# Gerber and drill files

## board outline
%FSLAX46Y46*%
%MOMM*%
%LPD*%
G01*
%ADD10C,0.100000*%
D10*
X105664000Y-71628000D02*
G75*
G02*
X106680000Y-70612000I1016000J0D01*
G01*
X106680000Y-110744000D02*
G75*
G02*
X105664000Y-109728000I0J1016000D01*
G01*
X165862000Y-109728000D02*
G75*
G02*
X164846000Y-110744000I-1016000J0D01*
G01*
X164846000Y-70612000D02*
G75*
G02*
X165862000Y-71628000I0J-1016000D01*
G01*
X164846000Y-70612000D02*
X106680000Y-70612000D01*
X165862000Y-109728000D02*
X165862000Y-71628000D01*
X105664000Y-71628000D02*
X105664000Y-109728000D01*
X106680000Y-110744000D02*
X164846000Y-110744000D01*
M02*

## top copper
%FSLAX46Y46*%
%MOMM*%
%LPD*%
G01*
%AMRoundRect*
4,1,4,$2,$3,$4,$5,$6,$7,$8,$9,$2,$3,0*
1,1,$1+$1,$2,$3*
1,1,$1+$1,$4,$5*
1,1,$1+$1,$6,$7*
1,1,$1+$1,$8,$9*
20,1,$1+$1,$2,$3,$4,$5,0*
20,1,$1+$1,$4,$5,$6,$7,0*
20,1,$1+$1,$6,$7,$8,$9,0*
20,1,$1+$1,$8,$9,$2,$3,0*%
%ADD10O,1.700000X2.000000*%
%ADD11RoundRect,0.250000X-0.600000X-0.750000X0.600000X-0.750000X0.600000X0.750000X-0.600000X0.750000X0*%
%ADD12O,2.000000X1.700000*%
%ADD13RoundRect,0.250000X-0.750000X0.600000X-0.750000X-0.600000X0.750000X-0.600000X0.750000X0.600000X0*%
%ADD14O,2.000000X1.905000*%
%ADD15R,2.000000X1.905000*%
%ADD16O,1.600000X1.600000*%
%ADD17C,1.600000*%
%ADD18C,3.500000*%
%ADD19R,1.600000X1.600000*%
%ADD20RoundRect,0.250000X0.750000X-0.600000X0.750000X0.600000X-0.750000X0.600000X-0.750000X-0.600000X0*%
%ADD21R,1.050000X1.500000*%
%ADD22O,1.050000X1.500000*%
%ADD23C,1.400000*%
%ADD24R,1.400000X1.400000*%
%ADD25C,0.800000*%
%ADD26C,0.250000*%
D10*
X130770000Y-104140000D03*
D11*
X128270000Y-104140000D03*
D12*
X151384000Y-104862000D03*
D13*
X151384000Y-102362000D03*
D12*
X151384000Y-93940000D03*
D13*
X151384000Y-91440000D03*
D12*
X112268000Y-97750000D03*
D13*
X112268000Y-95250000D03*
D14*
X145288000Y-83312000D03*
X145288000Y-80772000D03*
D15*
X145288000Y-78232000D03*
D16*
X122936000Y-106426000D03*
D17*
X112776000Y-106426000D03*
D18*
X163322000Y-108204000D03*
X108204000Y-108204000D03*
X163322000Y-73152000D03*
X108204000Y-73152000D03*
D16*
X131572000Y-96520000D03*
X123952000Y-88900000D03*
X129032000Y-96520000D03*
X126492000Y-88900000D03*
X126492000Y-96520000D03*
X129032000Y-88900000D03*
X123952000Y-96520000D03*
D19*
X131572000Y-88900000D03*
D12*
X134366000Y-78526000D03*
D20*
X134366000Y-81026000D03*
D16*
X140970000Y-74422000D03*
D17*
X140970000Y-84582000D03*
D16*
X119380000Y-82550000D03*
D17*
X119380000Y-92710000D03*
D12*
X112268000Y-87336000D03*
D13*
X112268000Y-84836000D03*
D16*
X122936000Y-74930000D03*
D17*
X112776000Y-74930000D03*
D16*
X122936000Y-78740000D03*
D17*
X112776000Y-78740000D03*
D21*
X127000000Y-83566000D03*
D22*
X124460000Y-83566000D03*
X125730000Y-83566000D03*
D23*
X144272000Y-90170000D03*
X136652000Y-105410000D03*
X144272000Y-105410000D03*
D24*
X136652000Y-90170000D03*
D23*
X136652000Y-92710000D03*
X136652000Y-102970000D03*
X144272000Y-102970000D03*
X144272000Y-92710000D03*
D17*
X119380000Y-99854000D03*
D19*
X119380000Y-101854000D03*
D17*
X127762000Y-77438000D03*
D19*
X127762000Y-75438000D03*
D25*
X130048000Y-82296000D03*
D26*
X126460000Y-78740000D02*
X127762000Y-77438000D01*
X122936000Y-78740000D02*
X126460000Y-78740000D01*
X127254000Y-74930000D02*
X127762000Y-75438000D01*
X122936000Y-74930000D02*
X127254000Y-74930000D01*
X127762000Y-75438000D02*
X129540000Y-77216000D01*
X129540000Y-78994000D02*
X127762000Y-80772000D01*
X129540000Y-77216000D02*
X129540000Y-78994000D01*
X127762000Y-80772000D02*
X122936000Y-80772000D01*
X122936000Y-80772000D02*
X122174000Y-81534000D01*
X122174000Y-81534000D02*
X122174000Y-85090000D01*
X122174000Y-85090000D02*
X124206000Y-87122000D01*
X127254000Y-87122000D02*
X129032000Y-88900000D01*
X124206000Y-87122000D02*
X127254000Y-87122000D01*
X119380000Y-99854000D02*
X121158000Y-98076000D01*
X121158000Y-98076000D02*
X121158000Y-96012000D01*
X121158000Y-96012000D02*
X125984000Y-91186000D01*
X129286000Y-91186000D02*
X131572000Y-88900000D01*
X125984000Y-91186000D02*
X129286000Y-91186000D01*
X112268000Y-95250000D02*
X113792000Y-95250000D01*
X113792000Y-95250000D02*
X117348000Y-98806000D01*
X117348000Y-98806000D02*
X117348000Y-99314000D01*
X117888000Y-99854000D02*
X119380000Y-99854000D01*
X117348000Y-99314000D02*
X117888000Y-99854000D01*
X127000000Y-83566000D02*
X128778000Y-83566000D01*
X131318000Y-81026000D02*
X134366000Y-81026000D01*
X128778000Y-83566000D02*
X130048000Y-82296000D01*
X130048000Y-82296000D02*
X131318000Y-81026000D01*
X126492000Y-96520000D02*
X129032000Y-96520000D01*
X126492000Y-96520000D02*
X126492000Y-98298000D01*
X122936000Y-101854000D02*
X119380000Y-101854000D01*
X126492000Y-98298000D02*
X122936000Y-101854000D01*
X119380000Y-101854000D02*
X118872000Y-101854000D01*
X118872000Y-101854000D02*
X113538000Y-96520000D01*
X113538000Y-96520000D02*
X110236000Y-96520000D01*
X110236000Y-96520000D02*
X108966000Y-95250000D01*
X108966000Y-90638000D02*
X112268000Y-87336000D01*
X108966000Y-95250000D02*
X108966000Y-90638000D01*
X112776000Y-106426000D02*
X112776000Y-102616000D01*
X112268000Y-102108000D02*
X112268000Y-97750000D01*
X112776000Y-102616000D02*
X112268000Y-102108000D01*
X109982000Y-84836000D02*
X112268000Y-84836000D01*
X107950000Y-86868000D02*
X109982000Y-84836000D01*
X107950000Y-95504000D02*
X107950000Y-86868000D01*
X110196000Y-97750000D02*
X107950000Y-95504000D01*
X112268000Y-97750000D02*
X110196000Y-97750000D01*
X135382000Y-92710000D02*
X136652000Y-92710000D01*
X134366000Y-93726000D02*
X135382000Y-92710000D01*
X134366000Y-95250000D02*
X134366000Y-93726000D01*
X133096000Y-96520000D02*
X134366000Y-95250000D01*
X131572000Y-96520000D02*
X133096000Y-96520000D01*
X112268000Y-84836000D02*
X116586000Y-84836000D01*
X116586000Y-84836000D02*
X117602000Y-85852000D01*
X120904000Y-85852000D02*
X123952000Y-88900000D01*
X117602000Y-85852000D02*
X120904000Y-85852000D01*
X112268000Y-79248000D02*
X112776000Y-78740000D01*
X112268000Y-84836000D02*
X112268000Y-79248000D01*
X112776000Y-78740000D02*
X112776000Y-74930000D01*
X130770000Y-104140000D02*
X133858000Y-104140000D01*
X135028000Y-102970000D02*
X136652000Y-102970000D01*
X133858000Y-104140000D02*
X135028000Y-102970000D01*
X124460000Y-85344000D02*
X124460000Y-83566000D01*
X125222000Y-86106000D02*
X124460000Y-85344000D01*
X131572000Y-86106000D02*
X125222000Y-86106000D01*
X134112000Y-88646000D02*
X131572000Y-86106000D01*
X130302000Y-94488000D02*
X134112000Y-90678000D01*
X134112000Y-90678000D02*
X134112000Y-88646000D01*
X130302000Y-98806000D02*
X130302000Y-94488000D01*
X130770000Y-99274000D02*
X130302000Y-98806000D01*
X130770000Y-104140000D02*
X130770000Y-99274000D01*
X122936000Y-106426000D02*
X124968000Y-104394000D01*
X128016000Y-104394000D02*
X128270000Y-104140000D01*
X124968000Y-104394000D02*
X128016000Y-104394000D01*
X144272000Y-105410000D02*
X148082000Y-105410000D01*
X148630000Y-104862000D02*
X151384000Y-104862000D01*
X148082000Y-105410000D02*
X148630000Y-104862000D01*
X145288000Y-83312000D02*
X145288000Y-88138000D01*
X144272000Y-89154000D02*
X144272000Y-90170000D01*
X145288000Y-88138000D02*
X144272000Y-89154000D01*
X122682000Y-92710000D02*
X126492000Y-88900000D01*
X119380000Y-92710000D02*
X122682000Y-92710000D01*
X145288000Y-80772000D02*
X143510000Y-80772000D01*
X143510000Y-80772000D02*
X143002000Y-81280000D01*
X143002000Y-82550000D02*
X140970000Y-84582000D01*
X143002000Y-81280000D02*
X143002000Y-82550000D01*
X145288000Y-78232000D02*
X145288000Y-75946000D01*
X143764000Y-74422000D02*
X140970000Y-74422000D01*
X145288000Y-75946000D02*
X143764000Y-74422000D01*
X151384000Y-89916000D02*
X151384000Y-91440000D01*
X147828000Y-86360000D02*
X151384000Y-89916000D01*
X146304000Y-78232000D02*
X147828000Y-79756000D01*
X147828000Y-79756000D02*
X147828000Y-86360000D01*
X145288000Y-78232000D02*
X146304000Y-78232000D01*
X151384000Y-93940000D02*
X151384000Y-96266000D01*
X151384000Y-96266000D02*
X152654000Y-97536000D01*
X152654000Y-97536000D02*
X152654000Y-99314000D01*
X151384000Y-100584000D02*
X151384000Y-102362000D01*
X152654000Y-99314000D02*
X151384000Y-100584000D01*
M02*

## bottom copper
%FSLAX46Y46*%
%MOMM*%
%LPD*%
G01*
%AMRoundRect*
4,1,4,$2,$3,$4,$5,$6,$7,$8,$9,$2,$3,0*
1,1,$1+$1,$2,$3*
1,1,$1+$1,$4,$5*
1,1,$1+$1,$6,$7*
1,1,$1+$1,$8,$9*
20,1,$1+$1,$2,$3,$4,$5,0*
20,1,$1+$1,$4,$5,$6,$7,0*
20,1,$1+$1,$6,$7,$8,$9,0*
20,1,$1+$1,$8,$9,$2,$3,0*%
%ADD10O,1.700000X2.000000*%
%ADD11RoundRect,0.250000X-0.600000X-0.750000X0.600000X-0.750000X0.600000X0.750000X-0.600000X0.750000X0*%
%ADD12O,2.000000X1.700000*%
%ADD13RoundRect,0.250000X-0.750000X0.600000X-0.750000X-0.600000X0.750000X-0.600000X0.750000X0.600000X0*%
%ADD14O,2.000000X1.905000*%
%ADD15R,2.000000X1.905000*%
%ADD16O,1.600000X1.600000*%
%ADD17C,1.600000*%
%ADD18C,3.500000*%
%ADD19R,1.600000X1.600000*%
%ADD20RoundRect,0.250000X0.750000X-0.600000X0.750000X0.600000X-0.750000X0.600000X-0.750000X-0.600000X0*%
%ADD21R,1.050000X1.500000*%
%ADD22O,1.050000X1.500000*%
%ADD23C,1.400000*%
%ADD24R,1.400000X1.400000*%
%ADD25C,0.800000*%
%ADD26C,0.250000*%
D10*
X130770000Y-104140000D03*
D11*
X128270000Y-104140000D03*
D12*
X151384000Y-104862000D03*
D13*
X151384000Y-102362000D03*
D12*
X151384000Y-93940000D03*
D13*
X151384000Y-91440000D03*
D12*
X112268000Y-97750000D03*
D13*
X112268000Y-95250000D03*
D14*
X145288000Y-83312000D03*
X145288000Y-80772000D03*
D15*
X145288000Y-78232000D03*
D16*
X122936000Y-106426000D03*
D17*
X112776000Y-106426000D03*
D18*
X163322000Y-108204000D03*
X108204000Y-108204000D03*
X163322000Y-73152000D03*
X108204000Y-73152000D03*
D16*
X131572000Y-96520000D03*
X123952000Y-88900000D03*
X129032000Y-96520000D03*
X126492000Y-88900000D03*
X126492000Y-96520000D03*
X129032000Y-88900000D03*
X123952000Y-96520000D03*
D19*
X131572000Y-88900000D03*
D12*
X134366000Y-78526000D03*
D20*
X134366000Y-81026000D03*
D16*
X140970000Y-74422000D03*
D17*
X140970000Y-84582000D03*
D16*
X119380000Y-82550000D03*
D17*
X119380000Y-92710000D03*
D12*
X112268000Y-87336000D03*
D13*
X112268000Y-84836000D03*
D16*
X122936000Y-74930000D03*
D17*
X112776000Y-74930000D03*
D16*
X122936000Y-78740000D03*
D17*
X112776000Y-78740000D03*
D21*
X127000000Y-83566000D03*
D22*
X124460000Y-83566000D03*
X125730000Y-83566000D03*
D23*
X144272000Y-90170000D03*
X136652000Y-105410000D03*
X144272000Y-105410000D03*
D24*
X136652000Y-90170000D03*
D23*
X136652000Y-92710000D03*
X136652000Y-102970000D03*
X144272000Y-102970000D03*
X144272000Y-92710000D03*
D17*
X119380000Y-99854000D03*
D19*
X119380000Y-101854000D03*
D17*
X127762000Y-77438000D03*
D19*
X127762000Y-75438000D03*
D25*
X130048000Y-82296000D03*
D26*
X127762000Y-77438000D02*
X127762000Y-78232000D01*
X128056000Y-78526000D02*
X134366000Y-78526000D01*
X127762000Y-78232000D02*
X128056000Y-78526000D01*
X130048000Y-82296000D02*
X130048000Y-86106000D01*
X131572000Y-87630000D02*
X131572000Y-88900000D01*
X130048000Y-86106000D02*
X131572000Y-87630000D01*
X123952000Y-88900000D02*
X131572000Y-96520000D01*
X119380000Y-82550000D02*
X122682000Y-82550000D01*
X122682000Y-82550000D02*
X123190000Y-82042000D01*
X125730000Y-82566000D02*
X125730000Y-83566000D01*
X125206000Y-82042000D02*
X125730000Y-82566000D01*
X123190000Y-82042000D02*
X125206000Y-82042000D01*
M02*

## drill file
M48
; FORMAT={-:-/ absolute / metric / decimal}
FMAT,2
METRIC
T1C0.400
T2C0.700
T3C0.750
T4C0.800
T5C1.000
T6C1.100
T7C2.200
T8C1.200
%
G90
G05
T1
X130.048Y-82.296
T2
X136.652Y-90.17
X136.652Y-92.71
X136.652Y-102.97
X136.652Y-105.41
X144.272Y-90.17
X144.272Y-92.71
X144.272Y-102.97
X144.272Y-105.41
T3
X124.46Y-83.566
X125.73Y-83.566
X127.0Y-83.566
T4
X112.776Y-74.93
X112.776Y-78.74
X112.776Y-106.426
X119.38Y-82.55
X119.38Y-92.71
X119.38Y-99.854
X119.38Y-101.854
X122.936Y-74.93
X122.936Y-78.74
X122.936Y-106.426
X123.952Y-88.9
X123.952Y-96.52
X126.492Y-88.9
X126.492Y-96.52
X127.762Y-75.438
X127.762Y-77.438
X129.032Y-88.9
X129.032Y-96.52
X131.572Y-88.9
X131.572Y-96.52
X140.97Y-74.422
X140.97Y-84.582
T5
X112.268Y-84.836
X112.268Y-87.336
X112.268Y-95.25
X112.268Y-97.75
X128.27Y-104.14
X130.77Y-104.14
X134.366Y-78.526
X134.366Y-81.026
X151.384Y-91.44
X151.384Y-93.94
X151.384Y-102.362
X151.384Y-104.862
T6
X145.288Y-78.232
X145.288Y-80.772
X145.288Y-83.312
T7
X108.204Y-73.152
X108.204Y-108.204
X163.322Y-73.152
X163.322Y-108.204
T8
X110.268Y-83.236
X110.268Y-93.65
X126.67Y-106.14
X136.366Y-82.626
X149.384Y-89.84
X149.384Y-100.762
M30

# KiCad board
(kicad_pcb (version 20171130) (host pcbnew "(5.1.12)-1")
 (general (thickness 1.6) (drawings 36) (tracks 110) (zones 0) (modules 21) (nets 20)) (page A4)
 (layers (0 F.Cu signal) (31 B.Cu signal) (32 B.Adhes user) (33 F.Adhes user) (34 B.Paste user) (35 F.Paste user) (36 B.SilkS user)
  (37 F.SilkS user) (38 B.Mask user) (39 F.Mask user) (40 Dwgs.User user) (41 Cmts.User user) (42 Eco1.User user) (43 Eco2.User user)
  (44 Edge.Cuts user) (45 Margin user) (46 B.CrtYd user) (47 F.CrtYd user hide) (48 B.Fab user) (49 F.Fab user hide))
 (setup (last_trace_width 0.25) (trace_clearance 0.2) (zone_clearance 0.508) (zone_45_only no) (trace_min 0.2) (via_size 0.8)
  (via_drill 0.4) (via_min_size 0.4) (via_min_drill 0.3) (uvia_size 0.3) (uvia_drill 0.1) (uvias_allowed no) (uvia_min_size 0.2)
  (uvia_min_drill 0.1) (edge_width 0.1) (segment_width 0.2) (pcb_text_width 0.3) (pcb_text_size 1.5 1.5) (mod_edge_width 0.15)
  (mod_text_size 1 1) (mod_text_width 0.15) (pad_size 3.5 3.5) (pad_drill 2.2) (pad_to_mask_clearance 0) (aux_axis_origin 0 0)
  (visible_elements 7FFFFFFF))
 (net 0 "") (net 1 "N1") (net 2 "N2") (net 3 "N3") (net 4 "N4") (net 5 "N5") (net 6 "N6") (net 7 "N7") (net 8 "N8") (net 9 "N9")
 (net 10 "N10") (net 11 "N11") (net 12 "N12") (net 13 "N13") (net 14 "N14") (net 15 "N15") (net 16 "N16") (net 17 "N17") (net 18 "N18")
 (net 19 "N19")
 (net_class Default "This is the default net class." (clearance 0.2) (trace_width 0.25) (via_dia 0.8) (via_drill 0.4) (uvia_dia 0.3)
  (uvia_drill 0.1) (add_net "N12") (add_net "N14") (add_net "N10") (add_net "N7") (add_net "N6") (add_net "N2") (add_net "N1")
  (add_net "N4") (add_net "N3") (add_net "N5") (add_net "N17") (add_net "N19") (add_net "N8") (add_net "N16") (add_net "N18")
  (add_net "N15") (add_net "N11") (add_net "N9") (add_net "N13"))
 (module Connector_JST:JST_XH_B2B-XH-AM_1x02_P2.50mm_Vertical (layer F.Cu) (at 128.27 104.14)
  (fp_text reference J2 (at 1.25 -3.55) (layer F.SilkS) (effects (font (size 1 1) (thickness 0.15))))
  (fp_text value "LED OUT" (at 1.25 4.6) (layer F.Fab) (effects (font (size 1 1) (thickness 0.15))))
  (pad "" np_thru_hole circle (at -1.6 2) (size 1.2 1.2) (drill 1.2) (layers *.Cu *.Mask))
  (pad 2 thru_hole oval (at 2.5 0) (size 1.7 2) (drill 1) (layers *.Cu *.Mask) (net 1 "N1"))
  (pad 1 thru_hole roundrect (at 0 0) (size 1.7 2) (drill 1) (layers *.Cu *.Mask) (roundrect_rratio 0.147059) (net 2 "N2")))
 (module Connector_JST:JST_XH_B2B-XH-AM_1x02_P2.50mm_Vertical (layer F.Cu) (at 151.384 102.362 270)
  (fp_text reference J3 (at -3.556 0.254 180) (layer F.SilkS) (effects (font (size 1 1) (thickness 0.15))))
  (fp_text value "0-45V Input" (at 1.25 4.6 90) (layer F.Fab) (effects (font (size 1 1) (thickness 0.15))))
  (pad "" np_thru_hole circle (at -1.6 2 270) (size 1.2 1.2) (drill 1.2) (layers *.Cu *.Mask))
  (pad 2 thru_hole oval (at 2.5 0 270) (size 1.7 2) (drill 1) (layers *.Cu *.Mask) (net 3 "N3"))
  (pad 1 thru_hole roundrect (at 0 0 270) (size 1.7 2) (drill 1) (layers *.Cu *.Mask) (roundrect_rratio 0.147059) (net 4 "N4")))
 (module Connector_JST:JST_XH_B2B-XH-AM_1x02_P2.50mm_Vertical (layer F.Cu) (at 151.384 91.44 270)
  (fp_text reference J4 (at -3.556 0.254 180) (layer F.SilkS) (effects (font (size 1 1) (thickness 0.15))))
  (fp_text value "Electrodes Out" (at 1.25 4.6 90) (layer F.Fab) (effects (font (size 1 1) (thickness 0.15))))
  (pad "" np_thru_hole circle (at -1.6 2 270) (size 1.2 1.2) (drill 1.2) (layers *.Cu *.Mask))
  (pad 2 thru_hole oval (at 2.5 0 270) (size 1.7 2) (drill 1) (layers *.Cu *.Mask) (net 4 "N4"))
  (pad 1 thru_hole roundrect (at 0 0 270) (size 1.7 2) (drill 1) (layers *.Cu *.Mask) (roundrect_rratio 0.147059) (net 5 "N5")))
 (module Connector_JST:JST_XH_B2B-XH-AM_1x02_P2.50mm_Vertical (layer F.Cu) (at 112.268 95.25 270)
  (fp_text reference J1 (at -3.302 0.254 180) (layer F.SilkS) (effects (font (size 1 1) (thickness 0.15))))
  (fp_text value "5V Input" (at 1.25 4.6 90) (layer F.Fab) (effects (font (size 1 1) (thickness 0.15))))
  (pad "" np_thru_hole circle (at -1.6 2 270) (size 1.2 1.2) (drill 1.2) (layers *.Cu *.Mask))
  (pad 2 thru_hole oval (at 2.5 0 270) (size 1.7 2) (drill 1) (layers *.Cu *.Mask) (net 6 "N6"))
  (pad 1 thru_hole roundrect (at 0 0 270) (size 1.7 2) (drill 1) (layers *.Cu *.Mask) (roundrect_rratio 0.147059) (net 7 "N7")))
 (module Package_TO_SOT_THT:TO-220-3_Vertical (layer F.Cu) (at 145.288 78.232 270)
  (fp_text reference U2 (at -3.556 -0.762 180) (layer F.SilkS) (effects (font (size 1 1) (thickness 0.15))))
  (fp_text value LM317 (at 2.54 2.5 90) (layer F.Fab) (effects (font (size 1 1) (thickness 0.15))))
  (pad 3 thru_hole oval (at 5.08 0 270) (size 1.905 2) (drill 1.1) (layers *.Cu *.Mask) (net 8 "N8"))
  (pad 2 thru_hole oval (at 2.54 0 270) (size 1.905 2) (drill 1.1) (layers *.Cu *.Mask) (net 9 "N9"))
  (pad 1 thru_hole rect (at 0 0 270) (size 1.905 2) (drill 1.1) (layers *.Cu *.Mask) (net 5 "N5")))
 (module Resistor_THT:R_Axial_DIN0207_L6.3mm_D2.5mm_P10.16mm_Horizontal (layer F.Cu) (at 112.776 106.426)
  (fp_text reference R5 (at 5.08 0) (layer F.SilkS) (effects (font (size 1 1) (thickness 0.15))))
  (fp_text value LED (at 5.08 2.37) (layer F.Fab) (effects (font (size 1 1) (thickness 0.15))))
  (pad 2 thru_hole oval (at 10.16 0) (size 1.6 1.6) (drill 0.8) (layers *.Cu *.Mask) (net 2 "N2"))
  (pad 1 thru_hole circle (at 0 0) (size 1.6 1.6) (drill 0.8) (layers *.Cu *.Mask) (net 6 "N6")))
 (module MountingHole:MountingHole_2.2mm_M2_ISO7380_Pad (layer F.Cu) (at 163.322 108.204)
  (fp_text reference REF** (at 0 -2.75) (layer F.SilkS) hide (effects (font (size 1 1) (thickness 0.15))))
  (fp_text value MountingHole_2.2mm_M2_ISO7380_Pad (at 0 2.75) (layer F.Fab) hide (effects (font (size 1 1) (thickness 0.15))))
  (pad 1 thru_hole circle (at 0 0) (size 3.5 3.5) (drill 2.2) (layers *.Cu *.Mask)))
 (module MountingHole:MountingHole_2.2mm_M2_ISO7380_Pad (layer F.Cu) (at 108.204 108.204)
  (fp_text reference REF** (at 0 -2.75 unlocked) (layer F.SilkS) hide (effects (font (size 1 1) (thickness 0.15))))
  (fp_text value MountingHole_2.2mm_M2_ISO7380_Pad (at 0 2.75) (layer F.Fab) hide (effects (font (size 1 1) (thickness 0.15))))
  (pad 1 thru_hole circle (at 0 0) (size 3.5 3.5) (drill 2.2) (layers *.Cu *.Mask)))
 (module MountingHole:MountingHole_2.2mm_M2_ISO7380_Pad (layer F.Cu) (at 163.322 73.152)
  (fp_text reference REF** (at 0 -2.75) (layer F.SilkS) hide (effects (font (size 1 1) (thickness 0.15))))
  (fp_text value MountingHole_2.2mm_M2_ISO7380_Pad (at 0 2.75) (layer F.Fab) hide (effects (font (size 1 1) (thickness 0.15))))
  (pad 1 thru_hole circle (at 0 0) (size 3.5 3.5) (drill 2.2) (layers *.Cu *.Mask)))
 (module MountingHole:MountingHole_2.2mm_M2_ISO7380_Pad (layer F.Cu) (at 108.204 73.152)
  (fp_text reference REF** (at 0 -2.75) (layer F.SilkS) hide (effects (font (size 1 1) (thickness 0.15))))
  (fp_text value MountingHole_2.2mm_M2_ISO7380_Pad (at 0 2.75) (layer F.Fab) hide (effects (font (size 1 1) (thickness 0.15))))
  (pad 1 thru_hole circle (at 0 0) (size 3.5 3.5) (drill 2.2) (layers *.Cu *.Mask)))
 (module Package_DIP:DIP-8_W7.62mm (layer F.Cu) (at 131.572 88.9 270)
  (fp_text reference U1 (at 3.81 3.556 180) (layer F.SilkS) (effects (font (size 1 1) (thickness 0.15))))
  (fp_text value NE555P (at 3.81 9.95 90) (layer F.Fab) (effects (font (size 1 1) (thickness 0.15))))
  (pad 8 thru_hole oval (at 7.62 0 270) (size 1.6 1.6) (drill 0.8) (layers *.Cu *.Mask) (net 6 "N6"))
  (pad 4 thru_hole oval (at 0 7.62 270) (size 1.6 1.6) (drill 0.8) (layers *.Cu *.Mask) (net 6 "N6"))
  (pad 7 thru_hole oval (at 7.62 2.54 270) (size 1.6 1.6) (drill 0.8) (layers *.Cu *.Mask) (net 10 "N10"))
  (pad 3 thru_hole oval (at 0 5.08 270) (size 1.6 1.6) (drill 0.8) (layers *.Cu *.Mask) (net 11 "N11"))
  (pad 6 thru_hole oval (at 7.62 5.08 270) (size 1.6 1.6) (drill 0.8) (layers *.Cu *.Mask) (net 10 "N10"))
  (pad 2 thru_hole oval (at 0 2.54 270) (size 1.6 1.6) (drill 0.8) (layers *.Cu *.Mask) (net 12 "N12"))
  (pad 5 thru_hole oval (at 7.62 7.62 270) (size 1.6 1.6) (drill 0.8) (layers *.Cu *.Mask) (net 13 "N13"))
  (pad 1 thru_hole rect (at 0 0 270) (size 1.6 1.6) (drill 0.8) (layers *.Cu *.Mask) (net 7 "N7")))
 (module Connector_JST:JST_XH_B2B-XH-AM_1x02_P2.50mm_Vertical (layer F.Cu) (at 134.366 81.026 90)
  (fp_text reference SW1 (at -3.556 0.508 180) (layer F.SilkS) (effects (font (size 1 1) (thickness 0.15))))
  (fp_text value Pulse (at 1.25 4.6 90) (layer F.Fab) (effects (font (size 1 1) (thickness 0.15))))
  (pad "" np_thru_hole circle (at -1.6 2 90) (size 1.2 1.2) (drill 1.2) (layers *.Cu *.Mask))
  (pad 2 thru_hole oval (at 2.5 0 90) (size 1.7 2) (drill 1) (layers *.Cu *.Mask) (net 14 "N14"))
  (pad 1 thru_hole roundrect (at 0 0 90) (size 1.7 2) (drill 1) (layers *.Cu *.Mask) (roundrect_rratio 0.147059) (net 7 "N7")))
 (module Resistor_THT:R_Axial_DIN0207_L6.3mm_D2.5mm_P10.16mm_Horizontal (layer F.Cu) (at 140.97 84.582 90)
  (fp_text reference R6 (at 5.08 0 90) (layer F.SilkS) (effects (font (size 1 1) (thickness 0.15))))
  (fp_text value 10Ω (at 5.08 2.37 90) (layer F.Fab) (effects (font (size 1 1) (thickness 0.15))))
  (pad 2 thru_hole oval (at 10.16 0 90) (size 1.6 1.6) (drill 0.8) (layers *.Cu *.Mask) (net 5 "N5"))
  (pad 1 thru_hole circle (at 0 0 90) (size 1.6 1.6) (drill 0.8) (layers *.Cu *.Mask) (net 9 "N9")))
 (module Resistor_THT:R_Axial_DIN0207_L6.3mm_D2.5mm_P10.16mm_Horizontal (layer F.Cu) (at 119.38 92.71 90)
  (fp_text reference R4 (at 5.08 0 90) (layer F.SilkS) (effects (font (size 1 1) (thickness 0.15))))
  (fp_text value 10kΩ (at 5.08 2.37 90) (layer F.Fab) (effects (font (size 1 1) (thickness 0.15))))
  (pad 2 thru_hole oval (at 10.16 0 90) (size 1.6 1.6) (drill 0.8) (layers *.Cu *.Mask) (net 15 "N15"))
  (pad 1 thru_hole circle (at 0 0 90) (size 1.6 1.6) (drill 0.8) (layers *.Cu *.Mask) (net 11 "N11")))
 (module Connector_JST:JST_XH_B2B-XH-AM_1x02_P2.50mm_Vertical (layer F.Cu) (at 112.268 84.836 270)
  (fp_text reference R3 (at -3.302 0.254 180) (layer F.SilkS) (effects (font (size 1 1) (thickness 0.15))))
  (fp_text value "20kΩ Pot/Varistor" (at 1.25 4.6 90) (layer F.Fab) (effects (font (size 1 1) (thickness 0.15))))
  (pad "" np_thru_hole circle (at -1.6 2 270) (size 1.2 1.2) (drill 1.2) (layers *.Cu *.Mask))
  (pad 2 thru_hole oval (at 2.5 0 270) (size 1.7 2) (drill 1) (layers *.Cu *.Mask) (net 10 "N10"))
  (pad 1 thru_hole roundrect (at 0 0 270) (size 1.7 2) (drill 1) (layers *.Cu *.Mask) (roundrect_rratio 0.147059) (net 6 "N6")))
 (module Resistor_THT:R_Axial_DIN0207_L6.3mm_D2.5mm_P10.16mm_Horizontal (layer F.Cu) (at 112.776 74.93)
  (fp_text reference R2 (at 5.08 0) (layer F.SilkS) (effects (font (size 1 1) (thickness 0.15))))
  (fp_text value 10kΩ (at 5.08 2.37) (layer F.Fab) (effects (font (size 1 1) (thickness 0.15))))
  (pad 2 thru_hole oval (at 10.16 0) (size 1.6 1.6) (drill 0.8) (layers *.Cu *.Mask) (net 12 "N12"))
  (pad 1 thru_hole circle (at 0 0) (size 1.6 1.6) (drill 0.8) (layers *.Cu *.Mask) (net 6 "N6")))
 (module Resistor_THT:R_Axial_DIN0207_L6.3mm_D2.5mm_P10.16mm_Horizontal (layer F.Cu) (at 112.776 78.74)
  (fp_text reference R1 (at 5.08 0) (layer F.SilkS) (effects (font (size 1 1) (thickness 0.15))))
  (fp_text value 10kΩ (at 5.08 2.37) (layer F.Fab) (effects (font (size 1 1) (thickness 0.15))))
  (pad 2 thru_hole oval (at 10.16 0) (size 1.6 1.6) (drill 0.8) (layers *.Cu *.Mask) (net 14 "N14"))
  (pad 1 thru_hole circle (at 0 0) (size 1.6 1.6) (drill 0.8) (layers *.Cu *.Mask) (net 6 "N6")))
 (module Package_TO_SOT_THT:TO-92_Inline (layer F.Cu) (at 127 83.566 180)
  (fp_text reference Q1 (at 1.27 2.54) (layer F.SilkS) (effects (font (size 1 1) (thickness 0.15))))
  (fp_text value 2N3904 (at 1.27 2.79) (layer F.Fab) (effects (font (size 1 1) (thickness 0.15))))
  (pad 1 thru_hole rect (at 0 0 180) (size 1.05 1.5) (drill 0.75) (layers *.Cu *.Mask) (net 7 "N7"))
  (pad 3 thru_hole oval (at 2.54 0 180) (size 1.05 1.5) (drill 0.75) (layers *.Cu *.Mask) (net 1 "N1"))
  (pad 2 thru_hole oval (at 1.27 0 180) (size 1.05 1.5) (drill 0.75) (layers *.Cu *.Mask) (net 15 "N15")))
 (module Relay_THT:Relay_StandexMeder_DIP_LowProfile (layer F.Cu) (at 136.652 90.17)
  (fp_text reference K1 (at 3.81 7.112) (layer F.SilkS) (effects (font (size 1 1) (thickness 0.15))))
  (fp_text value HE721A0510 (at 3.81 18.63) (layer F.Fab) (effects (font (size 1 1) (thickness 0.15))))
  (pad 14 thru_hole circle (at 7.62 0) (size 1.4 1.4) (drill 0.7) (layers *.Cu *.Mask) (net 8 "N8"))
  (pad 7 thru_hole circle (at 0 15.24) (size 1.4 1.4) (drill 0.7) (layers *.Cu *.Mask) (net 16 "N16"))
  (pad 8 thru_hole circle (at 7.62 15.24) (size 1.4 1.4) (drill 0.7) (layers *.Cu *.Mask) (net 3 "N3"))
  (pad 1 thru_hole rect (at 0 0) (size 1.4 1.4) (drill 0.7) (layers *.Cu *.Mask) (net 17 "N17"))
  (pad 2 thru_hole circle (at 0 2.54) (size 1.4 1.4) (drill 0.7) (layers *.Cu *.Mask) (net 6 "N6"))
  (pad 6 thru_hole circle (at 0 12.8) (size 1.4 1.4) (drill 0.7) (layers *.Cu *.Mask) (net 1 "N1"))
  (pad 9 thru_hole circle (at 7.62 12.8) (size 1.4 1.4) (drill 0.7) (layers *.Cu *.Mask) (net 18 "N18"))
  (pad 13 thru_hole circle (at 7.62 2.54) (size 1.4 1.4) (drill 0.7) (layers *.Cu *.Mask) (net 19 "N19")))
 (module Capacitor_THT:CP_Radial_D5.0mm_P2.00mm (layer F.Cu) (at 119.38 101.854 90)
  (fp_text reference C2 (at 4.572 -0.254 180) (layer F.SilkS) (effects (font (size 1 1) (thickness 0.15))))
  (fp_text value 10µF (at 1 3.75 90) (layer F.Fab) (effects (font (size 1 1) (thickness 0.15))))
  (pad 2 thru_hole circle (at 2 0 90) (size 1.6 1.6) (drill 0.8) (layers *.Cu *.Mask) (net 7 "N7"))
  (pad 1 thru_hole rect (at 0 0 90) (size 1.6 1.6) (drill 0.8) (layers *.Cu *.Mask) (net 10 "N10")))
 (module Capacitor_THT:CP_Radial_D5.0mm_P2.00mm (layer F.Cu) (at 127.762 75.438 270)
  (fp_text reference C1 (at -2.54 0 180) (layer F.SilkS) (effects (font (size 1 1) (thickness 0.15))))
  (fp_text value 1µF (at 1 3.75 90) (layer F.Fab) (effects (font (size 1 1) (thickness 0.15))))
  (pad 2 thru_hole circle (at 2 0 270) (size 1.6 1.6) (drill 0.8) (layers *.Cu *.Mask) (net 14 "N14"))
  (pad 1 thru_hole rect (at 0 0 270) (size 1.6 1.6) (drill 0.8) (layers *.Cu *.Mask) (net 12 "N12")))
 (gr_arc (start 106.68 71.628) (end 106.68 70.612) (angle -90) (layer Edge.Cuts) (width 0.1))
 (gr_arc (start 106.68 109.728) (end 105.664 109.728) (angle -90) (layer Edge.Cuts) (width 0.1))
 (gr_arc (start 164.846 109.728) (end 164.846 110.744) (angle -90) (layer Edge.Cuts) (width 0.1))
 (gr_arc (start 164.846 71.628) (end 165.862 71.628) (angle -90) (layer Edge.Cuts) (width 0.1))
 (gr_line (start 164.846 70.612) (end 106.68 70.612) (layer Edge.Cuts) (width 0.1))
 (gr_line (start 165.862 109.728) (end 165.862 71.628) (layer Edge.Cuts) (width 0.1))
 (gr_line (start 105.664 71.628) (end 105.664 109.728) (layer Edge.Cuts) (width 0.1))
 (gr_line (start 106.68 110.744) (end 164.846 110.744) (layer Edge.Cuts) (width 0.1))
 (segment (start 126.46 78.74) (end 127.762 77.438) (width 0.25) (layer F.Cu) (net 14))
 (segment (start 122.936 78.74) (end 126.46 78.74) (width 0.25) (layer F.Cu) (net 14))
 (segment (start 127.762 77.438) (end 127.762 78.232) (width 0.25) (layer B.Cu) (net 14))
 (segment (start 128.056 78.526) (end 134.366 78.526) (width 0.25) (layer B.Cu) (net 14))
 (segment (start 127.762 78.232) (end 128.056 78.526) (width 0.25) (layer B.Cu) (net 14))
 (segment (start 127.254 74.93) (end 127.762 75.438) (width 0.25) (layer F.Cu) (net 12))
 (segment (start 122.936 74.93) (end 127.254 74.93) (width 0.25) (layer F.Cu) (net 12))
 (segment (start 127.762 75.438) (end 129.54 77.216) (width 0.25) (layer F.Cu) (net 12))
 (segment (start 129.54 78.994) (end 127.762 80.772) (width 0.25) (layer F.Cu) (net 12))
 (segment (start 129.54 77.216) (end 129.54 78.994) (width 0.25) (layer F.Cu) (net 12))
 (segment (start 127.762 80.772) (end 122.936 80.772) (width 0.25) (layer F.Cu) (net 12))
 (segment (start 122.936 80.772) (end 122.174 81.534) (width 0.25) (layer F.Cu) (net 12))
 (segment (start 122.174 81.534) (end 122.174 85.09) (width 0.25) (layer F.Cu) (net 12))
 (segment (start 122.174 85.09) (end 124.206 87.122) (width 0.25) (layer F.Cu) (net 12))
 (segment (start 127.254 87.122) (end 129.032 88.9) (width 0.25) (layer F.Cu) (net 12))
 (segment (start 124.206 87.122) (end 127.254 87.122) (width 0.25) (layer F.Cu) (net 12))
 (segment (start 119.38 99.854) (end 121.158 98.076) (width 0.25) (layer F.Cu) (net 7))
 (segment (start 121.158 98.076) (end 121.158 96.012) (width 0.25) (layer F.Cu) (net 7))
 (segment (start 121.158 96.012) (end 125.984 91.186) (width 0.25) (layer F.Cu) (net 7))
 (segment (start 129.286 91.186) (end 131.572 88.9) (width 0.25) (layer F.Cu) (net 7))
 (segment (start 125.984 91.186) (end 129.286 91.186) (width 0.25) (layer F.Cu) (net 7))
 (segment (start 112.268 95.25) (end 113.792 95.25) (width 0.25) (layer F.Cu) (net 7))
 (segment (start 113.792 95.25) (end 117.348 98.806) (width 0.25) (layer F.Cu) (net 7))
 (segment (start 117.348 98.806) (end 117.348 99.314) (width 0.25) (layer F.Cu) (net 7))
 (segment (start 117.888 99.854) (end 119.38 99.854) (width 0.25) (layer F.Cu) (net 7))
 (segment (start 117.348 99.314) (end 117.888 99.854) (width 0.25) (layer F.Cu) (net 7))
 (segment (start 127 83.566) (end 128.778 83.566) (width 0.25) (layer F.Cu) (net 7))
 (segment (start 131.318 81.026) (end 134.366 81.026) (width 0.25) (layer F.Cu) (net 7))
 (segment (start 128.778 83.566) (end 130.048 82.296) (width 0.25) (layer F.Cu) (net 7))
 (segment (start 130.048 82.296) (end 131.318 81.026) (width 0.25) (layer F.Cu) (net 7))
 (via (at 130.048 82.296) (size 0.8) (drill 0.4) (layers F.Cu B.Cu) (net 7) (status 1000000))
 (segment (start 130.048 82.296) (end 130.048 86.106) (width 0.25) (layer B.Cu) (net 7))
 (segment (start 131.572 87.63) (end 131.572 88.9) (width 0.25) (layer B.Cu) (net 7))
 (segment (start 130.048 86.106) (end 131.572 87.63) (width 0.25) (layer B.Cu) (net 7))
 (segment (start 126.492 96.52) (end 129.032 96.52) (width 0.25) (layer F.Cu) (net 10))
 (segment (start 126.492 96.52) (end 126.492 98.298) (width 0.25) (layer F.Cu) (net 10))
 (segment (start 122.936 101.854) (end 119.38 101.854) (width 0.25) (layer F.Cu) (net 10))
 (segment (start 126.492 98.298) (end 122.936 101.854) (width 0.25) (layer F.Cu) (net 10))
 (segment (start 119.38 101.854) (end 118.872 101.854) (width 0.25) (layer F.Cu) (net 10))
 (segment (start 118.872 101.854) (end 113.538 96.52) (width 0.25) (layer F.Cu) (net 10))
 (segment (start 113.538 96.52) (end 110.236 96.52) (width 0.25) (layer F.Cu) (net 10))
 (segment (start 110.236 96.52) (end 108.966 95.25) (width 0.25) (layer F.Cu) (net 10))
 (segment (start 108.966 90.638) (end 112.268 87.336) (width 0.25) (layer F.Cu) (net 10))
 (segment (start 108.966 95.25) (end 108.966 90.638) (width 0.25) (layer F.Cu) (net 10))
 (segment (start 112.776 106.426) (end 112.776 102.616) (width 0.25) (layer F.Cu) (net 6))
 (segment (start 112.268 102.108) (end 112.268 97.75) (width 0.25) (layer F.Cu) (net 6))
 (segment (start 112.776 102.616) (end 112.268 102.108) (width 0.25) (layer F.Cu) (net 6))
 (segment (start 109.982 84.836) (end 112.268 84.836) (width 0.25) (layer F.Cu) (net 6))
 (segment (start 107.95 86.868) (end 109.982 84.836) (width 0.25) (layer F.Cu) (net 6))
 (segment (start 107.95 95.504) (end 107.95 86.868) (width 0.25) (layer F.Cu) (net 6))
 (segment (start 110.196 97.75) (end 107.95 95.504) (width 0.25) (layer F.Cu) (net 6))
 (segment (start 112.268 97.75) (end 110.196 97.75) (width 0.25) (layer F.Cu) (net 6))
 (segment (start 135.382 92.71) (end 136.652 92.71) (width 0.25) (layer F.Cu) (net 6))
 (segment (start 134.366 93.726) (end 135.382 92.71) (width 0.25) (layer F.Cu) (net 6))
 (segment (start 134.366 95.25) (end 134.366 93.726) (width 0.25) (layer F.Cu) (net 6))
 (segment (start 133.096 96.52) (end 134.366 95.25) (width 0.25) (layer F.Cu) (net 6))
 (segment (start 131.572 96.52) (end 133.096 96.52) (width 0.25) (layer F.Cu) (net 6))
 (segment (start 112.268 84.836) (end 116.586 84.836) (width 0.25) (layer F.Cu) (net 6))
 (segment (start 116.586 84.836) (end 117.602 85.852) (width 0.25) (layer F.Cu) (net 6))
 (segment (start 120.904 85.852) (end 123.952 88.9) (width 0.25) (layer F.Cu) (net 6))
 (segment (start 117.602 85.852) (end 120.904 85.852) (width 0.25) (layer F.Cu) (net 6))
 (segment (start 112.268 79.248) (end 112.776 78.74) (width 0.25) (layer F.Cu) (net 6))
 (segment (start 112.268 84.836) (end 112.268 79.248) (width 0.25) (layer F.Cu) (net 6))
 (segment (start 112.776 78.74) (end 112.776 74.93) (width 0.25) (layer F.Cu) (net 6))
 (segment (start 123.952 88.9) (end 131.572 96.52) (width 0.25) (layer B.Cu) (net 6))
 (segment (start 130.77 104.14) (end 133.858 104.14) (width 0.25) (layer F.Cu) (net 1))
 (segment (start 135.028 102.97) (end 136.652 102.97) (width 0.25) (layer F.Cu) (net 1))
 (segment (start 133.858 104.14) (end 135.028 102.97) (width 0.25) (layer F.Cu) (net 1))
 (segment (start 124.46 85.344) (end 124.46 83.566) (width 0.25) (layer F.Cu) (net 1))
 (segment (start 125.222 86.106) (end 124.46 85.344) (width 0.25) (layer F.Cu) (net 1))
 (segment (start 131.572 86.106) (end 125.222 86.106) (width 0.25) (layer F.Cu) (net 1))
 (segment (start 134.112 88.646) (end 131.572 86.106) (width 0.25) (layer F.Cu) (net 1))
 (segment (start 130.302 94.488) (end 134.112 90.678) (width 0.25) (layer F.Cu) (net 1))
 (segment (start 134.112 90.678) (end 134.112 88.646) (width 0.25) (layer F.Cu) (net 1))
 (segment (start 130.302 98.806) (end 130.302 94.488) (width 0.25) (layer F.Cu) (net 1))
 (segment (start 130.77 99.274) (end 130.302 98.806) (width 0.25) (layer F.Cu) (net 1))
 (segment (start 130.77 104.14) (end 130.77 99.274) (width 0.25) (layer F.Cu) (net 1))
 (segment (start 122.936 106.426) (end 124.968 104.394) (width 0.25) (layer F.Cu) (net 2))
 (segment (start 128.016 104.394) (end 128.27 104.14) (width 0.25) (layer F.Cu) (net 2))
 (segment (start 124.968 104.394) (end 128.016 104.394) (width 0.25) (layer F.Cu) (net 2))
 (segment (start 144.272 105.41) (end 148.082 105.41) (width 0.25) (layer F.Cu) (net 3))
 (segment (start 148.63 104.862) (end 151.384 104.862) (width 0.25) (layer F.Cu) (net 3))
 (segment (start 148.082 105.41) (end 148.63 104.862) (width 0.25) (layer F.Cu) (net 3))
 (segment (start 145.288 83.312) (end 145.288 88.138) (width 0.25) (layer F.Cu) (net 8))
 (segment (start 144.272 89.154) (end 144.272 90.17) (width 0.25) (layer F.Cu) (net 8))
 (segment (start 145.288 88.138) (end 144.272 89.154) (width 0.25) (layer F.Cu) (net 8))
 (segment (start 119.38 82.55) (end 122.682 82.55) (width 0.25) (layer B.Cu) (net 15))
 (segment (start 122.682 82.55) (end 123.19 82.042) (width 0.25) (layer B.Cu) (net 15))
 (segment (start 125.73 82.566) (end 125.73 83.566) (width 0.25) (layer B.Cu) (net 15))
 (segment (start 125.206 82.042) (end 125.73 82.566) (width 0.25) (layer B.Cu) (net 15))
 (segment (start 123.19 82.042) (end 125.206 82.042) (width 0.25) (layer B.Cu) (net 15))
 (segment (start 122.682 92.71) (end 126.492 88.9) (width 0.25) (layer F.Cu) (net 11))
 (segment (start 119.38 92.71) (end 122.682 92.71) (width 0.25) (layer F.Cu) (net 11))
 (segment (start 145.288 80.772) (end 143.51 80.772) (width 0.25) (layer F.Cu) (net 9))
 (segment (start 143.51 80.772) (end 143.002 81.28) (width 0.25) (layer F.Cu) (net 9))
 (segment (start 143.002 82.55) (end 140.97 84.582) (width 0.25) (layer F.Cu) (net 9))
 (segment (start 143.002 81.28) (end 143.002 82.55) (width 0.25) (layer F.Cu) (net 9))
 (segment (start 145.288 78.232) (end 145.288 75.946) (width 0.25) (layer F.Cu) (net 5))
 (segment (start 143.764 74.422) (end 140.97 74.422) (width 0.25) (layer F.Cu) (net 5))
 (segment (start 145.288 75.946) (end 143.764 74.422) (width 0.25) (layer F.Cu) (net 5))
 (segment (start 151.384 89.916) (end 151.384 91.44) (width 0.25) (layer F.Cu) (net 5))
 (segment (start 147.828 86.36) (end 151.384 89.916) (width 0.25) (layer F.Cu) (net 5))
 (segment (start 146.304 78.232) (end 147.828 79.756) (width 0.25) (layer F.Cu) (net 5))
 (segment (start 147.828 79.756) (end 147.828 86.36) (width 0.25) (layer F.Cu) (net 5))
 (segment (start 145.288 78.232) (end 146.304 78.232) (width 0.25) (layer F.Cu) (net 5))
 (segment (start 151.384 93.94) (end 151.384 96.266) (width 0.25) (layer F.Cu) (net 4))
 (segment (start 151.384 96.266) (end 152.654 97.536) (width 0.25) (layer F.Cu) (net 4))
 (segment (start 152.654 97.536) (end 152.654 99.314) (width 0.25) (layer F.Cu) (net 4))
 (segment (start 151.384 100.584) (end 151.384 102.362) (width 0.25) (layer F.Cu) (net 4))
 (segment (start 152.654 99.314) (end 151.384 100.584) (width 0.25) (layer F.Cu) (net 4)))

